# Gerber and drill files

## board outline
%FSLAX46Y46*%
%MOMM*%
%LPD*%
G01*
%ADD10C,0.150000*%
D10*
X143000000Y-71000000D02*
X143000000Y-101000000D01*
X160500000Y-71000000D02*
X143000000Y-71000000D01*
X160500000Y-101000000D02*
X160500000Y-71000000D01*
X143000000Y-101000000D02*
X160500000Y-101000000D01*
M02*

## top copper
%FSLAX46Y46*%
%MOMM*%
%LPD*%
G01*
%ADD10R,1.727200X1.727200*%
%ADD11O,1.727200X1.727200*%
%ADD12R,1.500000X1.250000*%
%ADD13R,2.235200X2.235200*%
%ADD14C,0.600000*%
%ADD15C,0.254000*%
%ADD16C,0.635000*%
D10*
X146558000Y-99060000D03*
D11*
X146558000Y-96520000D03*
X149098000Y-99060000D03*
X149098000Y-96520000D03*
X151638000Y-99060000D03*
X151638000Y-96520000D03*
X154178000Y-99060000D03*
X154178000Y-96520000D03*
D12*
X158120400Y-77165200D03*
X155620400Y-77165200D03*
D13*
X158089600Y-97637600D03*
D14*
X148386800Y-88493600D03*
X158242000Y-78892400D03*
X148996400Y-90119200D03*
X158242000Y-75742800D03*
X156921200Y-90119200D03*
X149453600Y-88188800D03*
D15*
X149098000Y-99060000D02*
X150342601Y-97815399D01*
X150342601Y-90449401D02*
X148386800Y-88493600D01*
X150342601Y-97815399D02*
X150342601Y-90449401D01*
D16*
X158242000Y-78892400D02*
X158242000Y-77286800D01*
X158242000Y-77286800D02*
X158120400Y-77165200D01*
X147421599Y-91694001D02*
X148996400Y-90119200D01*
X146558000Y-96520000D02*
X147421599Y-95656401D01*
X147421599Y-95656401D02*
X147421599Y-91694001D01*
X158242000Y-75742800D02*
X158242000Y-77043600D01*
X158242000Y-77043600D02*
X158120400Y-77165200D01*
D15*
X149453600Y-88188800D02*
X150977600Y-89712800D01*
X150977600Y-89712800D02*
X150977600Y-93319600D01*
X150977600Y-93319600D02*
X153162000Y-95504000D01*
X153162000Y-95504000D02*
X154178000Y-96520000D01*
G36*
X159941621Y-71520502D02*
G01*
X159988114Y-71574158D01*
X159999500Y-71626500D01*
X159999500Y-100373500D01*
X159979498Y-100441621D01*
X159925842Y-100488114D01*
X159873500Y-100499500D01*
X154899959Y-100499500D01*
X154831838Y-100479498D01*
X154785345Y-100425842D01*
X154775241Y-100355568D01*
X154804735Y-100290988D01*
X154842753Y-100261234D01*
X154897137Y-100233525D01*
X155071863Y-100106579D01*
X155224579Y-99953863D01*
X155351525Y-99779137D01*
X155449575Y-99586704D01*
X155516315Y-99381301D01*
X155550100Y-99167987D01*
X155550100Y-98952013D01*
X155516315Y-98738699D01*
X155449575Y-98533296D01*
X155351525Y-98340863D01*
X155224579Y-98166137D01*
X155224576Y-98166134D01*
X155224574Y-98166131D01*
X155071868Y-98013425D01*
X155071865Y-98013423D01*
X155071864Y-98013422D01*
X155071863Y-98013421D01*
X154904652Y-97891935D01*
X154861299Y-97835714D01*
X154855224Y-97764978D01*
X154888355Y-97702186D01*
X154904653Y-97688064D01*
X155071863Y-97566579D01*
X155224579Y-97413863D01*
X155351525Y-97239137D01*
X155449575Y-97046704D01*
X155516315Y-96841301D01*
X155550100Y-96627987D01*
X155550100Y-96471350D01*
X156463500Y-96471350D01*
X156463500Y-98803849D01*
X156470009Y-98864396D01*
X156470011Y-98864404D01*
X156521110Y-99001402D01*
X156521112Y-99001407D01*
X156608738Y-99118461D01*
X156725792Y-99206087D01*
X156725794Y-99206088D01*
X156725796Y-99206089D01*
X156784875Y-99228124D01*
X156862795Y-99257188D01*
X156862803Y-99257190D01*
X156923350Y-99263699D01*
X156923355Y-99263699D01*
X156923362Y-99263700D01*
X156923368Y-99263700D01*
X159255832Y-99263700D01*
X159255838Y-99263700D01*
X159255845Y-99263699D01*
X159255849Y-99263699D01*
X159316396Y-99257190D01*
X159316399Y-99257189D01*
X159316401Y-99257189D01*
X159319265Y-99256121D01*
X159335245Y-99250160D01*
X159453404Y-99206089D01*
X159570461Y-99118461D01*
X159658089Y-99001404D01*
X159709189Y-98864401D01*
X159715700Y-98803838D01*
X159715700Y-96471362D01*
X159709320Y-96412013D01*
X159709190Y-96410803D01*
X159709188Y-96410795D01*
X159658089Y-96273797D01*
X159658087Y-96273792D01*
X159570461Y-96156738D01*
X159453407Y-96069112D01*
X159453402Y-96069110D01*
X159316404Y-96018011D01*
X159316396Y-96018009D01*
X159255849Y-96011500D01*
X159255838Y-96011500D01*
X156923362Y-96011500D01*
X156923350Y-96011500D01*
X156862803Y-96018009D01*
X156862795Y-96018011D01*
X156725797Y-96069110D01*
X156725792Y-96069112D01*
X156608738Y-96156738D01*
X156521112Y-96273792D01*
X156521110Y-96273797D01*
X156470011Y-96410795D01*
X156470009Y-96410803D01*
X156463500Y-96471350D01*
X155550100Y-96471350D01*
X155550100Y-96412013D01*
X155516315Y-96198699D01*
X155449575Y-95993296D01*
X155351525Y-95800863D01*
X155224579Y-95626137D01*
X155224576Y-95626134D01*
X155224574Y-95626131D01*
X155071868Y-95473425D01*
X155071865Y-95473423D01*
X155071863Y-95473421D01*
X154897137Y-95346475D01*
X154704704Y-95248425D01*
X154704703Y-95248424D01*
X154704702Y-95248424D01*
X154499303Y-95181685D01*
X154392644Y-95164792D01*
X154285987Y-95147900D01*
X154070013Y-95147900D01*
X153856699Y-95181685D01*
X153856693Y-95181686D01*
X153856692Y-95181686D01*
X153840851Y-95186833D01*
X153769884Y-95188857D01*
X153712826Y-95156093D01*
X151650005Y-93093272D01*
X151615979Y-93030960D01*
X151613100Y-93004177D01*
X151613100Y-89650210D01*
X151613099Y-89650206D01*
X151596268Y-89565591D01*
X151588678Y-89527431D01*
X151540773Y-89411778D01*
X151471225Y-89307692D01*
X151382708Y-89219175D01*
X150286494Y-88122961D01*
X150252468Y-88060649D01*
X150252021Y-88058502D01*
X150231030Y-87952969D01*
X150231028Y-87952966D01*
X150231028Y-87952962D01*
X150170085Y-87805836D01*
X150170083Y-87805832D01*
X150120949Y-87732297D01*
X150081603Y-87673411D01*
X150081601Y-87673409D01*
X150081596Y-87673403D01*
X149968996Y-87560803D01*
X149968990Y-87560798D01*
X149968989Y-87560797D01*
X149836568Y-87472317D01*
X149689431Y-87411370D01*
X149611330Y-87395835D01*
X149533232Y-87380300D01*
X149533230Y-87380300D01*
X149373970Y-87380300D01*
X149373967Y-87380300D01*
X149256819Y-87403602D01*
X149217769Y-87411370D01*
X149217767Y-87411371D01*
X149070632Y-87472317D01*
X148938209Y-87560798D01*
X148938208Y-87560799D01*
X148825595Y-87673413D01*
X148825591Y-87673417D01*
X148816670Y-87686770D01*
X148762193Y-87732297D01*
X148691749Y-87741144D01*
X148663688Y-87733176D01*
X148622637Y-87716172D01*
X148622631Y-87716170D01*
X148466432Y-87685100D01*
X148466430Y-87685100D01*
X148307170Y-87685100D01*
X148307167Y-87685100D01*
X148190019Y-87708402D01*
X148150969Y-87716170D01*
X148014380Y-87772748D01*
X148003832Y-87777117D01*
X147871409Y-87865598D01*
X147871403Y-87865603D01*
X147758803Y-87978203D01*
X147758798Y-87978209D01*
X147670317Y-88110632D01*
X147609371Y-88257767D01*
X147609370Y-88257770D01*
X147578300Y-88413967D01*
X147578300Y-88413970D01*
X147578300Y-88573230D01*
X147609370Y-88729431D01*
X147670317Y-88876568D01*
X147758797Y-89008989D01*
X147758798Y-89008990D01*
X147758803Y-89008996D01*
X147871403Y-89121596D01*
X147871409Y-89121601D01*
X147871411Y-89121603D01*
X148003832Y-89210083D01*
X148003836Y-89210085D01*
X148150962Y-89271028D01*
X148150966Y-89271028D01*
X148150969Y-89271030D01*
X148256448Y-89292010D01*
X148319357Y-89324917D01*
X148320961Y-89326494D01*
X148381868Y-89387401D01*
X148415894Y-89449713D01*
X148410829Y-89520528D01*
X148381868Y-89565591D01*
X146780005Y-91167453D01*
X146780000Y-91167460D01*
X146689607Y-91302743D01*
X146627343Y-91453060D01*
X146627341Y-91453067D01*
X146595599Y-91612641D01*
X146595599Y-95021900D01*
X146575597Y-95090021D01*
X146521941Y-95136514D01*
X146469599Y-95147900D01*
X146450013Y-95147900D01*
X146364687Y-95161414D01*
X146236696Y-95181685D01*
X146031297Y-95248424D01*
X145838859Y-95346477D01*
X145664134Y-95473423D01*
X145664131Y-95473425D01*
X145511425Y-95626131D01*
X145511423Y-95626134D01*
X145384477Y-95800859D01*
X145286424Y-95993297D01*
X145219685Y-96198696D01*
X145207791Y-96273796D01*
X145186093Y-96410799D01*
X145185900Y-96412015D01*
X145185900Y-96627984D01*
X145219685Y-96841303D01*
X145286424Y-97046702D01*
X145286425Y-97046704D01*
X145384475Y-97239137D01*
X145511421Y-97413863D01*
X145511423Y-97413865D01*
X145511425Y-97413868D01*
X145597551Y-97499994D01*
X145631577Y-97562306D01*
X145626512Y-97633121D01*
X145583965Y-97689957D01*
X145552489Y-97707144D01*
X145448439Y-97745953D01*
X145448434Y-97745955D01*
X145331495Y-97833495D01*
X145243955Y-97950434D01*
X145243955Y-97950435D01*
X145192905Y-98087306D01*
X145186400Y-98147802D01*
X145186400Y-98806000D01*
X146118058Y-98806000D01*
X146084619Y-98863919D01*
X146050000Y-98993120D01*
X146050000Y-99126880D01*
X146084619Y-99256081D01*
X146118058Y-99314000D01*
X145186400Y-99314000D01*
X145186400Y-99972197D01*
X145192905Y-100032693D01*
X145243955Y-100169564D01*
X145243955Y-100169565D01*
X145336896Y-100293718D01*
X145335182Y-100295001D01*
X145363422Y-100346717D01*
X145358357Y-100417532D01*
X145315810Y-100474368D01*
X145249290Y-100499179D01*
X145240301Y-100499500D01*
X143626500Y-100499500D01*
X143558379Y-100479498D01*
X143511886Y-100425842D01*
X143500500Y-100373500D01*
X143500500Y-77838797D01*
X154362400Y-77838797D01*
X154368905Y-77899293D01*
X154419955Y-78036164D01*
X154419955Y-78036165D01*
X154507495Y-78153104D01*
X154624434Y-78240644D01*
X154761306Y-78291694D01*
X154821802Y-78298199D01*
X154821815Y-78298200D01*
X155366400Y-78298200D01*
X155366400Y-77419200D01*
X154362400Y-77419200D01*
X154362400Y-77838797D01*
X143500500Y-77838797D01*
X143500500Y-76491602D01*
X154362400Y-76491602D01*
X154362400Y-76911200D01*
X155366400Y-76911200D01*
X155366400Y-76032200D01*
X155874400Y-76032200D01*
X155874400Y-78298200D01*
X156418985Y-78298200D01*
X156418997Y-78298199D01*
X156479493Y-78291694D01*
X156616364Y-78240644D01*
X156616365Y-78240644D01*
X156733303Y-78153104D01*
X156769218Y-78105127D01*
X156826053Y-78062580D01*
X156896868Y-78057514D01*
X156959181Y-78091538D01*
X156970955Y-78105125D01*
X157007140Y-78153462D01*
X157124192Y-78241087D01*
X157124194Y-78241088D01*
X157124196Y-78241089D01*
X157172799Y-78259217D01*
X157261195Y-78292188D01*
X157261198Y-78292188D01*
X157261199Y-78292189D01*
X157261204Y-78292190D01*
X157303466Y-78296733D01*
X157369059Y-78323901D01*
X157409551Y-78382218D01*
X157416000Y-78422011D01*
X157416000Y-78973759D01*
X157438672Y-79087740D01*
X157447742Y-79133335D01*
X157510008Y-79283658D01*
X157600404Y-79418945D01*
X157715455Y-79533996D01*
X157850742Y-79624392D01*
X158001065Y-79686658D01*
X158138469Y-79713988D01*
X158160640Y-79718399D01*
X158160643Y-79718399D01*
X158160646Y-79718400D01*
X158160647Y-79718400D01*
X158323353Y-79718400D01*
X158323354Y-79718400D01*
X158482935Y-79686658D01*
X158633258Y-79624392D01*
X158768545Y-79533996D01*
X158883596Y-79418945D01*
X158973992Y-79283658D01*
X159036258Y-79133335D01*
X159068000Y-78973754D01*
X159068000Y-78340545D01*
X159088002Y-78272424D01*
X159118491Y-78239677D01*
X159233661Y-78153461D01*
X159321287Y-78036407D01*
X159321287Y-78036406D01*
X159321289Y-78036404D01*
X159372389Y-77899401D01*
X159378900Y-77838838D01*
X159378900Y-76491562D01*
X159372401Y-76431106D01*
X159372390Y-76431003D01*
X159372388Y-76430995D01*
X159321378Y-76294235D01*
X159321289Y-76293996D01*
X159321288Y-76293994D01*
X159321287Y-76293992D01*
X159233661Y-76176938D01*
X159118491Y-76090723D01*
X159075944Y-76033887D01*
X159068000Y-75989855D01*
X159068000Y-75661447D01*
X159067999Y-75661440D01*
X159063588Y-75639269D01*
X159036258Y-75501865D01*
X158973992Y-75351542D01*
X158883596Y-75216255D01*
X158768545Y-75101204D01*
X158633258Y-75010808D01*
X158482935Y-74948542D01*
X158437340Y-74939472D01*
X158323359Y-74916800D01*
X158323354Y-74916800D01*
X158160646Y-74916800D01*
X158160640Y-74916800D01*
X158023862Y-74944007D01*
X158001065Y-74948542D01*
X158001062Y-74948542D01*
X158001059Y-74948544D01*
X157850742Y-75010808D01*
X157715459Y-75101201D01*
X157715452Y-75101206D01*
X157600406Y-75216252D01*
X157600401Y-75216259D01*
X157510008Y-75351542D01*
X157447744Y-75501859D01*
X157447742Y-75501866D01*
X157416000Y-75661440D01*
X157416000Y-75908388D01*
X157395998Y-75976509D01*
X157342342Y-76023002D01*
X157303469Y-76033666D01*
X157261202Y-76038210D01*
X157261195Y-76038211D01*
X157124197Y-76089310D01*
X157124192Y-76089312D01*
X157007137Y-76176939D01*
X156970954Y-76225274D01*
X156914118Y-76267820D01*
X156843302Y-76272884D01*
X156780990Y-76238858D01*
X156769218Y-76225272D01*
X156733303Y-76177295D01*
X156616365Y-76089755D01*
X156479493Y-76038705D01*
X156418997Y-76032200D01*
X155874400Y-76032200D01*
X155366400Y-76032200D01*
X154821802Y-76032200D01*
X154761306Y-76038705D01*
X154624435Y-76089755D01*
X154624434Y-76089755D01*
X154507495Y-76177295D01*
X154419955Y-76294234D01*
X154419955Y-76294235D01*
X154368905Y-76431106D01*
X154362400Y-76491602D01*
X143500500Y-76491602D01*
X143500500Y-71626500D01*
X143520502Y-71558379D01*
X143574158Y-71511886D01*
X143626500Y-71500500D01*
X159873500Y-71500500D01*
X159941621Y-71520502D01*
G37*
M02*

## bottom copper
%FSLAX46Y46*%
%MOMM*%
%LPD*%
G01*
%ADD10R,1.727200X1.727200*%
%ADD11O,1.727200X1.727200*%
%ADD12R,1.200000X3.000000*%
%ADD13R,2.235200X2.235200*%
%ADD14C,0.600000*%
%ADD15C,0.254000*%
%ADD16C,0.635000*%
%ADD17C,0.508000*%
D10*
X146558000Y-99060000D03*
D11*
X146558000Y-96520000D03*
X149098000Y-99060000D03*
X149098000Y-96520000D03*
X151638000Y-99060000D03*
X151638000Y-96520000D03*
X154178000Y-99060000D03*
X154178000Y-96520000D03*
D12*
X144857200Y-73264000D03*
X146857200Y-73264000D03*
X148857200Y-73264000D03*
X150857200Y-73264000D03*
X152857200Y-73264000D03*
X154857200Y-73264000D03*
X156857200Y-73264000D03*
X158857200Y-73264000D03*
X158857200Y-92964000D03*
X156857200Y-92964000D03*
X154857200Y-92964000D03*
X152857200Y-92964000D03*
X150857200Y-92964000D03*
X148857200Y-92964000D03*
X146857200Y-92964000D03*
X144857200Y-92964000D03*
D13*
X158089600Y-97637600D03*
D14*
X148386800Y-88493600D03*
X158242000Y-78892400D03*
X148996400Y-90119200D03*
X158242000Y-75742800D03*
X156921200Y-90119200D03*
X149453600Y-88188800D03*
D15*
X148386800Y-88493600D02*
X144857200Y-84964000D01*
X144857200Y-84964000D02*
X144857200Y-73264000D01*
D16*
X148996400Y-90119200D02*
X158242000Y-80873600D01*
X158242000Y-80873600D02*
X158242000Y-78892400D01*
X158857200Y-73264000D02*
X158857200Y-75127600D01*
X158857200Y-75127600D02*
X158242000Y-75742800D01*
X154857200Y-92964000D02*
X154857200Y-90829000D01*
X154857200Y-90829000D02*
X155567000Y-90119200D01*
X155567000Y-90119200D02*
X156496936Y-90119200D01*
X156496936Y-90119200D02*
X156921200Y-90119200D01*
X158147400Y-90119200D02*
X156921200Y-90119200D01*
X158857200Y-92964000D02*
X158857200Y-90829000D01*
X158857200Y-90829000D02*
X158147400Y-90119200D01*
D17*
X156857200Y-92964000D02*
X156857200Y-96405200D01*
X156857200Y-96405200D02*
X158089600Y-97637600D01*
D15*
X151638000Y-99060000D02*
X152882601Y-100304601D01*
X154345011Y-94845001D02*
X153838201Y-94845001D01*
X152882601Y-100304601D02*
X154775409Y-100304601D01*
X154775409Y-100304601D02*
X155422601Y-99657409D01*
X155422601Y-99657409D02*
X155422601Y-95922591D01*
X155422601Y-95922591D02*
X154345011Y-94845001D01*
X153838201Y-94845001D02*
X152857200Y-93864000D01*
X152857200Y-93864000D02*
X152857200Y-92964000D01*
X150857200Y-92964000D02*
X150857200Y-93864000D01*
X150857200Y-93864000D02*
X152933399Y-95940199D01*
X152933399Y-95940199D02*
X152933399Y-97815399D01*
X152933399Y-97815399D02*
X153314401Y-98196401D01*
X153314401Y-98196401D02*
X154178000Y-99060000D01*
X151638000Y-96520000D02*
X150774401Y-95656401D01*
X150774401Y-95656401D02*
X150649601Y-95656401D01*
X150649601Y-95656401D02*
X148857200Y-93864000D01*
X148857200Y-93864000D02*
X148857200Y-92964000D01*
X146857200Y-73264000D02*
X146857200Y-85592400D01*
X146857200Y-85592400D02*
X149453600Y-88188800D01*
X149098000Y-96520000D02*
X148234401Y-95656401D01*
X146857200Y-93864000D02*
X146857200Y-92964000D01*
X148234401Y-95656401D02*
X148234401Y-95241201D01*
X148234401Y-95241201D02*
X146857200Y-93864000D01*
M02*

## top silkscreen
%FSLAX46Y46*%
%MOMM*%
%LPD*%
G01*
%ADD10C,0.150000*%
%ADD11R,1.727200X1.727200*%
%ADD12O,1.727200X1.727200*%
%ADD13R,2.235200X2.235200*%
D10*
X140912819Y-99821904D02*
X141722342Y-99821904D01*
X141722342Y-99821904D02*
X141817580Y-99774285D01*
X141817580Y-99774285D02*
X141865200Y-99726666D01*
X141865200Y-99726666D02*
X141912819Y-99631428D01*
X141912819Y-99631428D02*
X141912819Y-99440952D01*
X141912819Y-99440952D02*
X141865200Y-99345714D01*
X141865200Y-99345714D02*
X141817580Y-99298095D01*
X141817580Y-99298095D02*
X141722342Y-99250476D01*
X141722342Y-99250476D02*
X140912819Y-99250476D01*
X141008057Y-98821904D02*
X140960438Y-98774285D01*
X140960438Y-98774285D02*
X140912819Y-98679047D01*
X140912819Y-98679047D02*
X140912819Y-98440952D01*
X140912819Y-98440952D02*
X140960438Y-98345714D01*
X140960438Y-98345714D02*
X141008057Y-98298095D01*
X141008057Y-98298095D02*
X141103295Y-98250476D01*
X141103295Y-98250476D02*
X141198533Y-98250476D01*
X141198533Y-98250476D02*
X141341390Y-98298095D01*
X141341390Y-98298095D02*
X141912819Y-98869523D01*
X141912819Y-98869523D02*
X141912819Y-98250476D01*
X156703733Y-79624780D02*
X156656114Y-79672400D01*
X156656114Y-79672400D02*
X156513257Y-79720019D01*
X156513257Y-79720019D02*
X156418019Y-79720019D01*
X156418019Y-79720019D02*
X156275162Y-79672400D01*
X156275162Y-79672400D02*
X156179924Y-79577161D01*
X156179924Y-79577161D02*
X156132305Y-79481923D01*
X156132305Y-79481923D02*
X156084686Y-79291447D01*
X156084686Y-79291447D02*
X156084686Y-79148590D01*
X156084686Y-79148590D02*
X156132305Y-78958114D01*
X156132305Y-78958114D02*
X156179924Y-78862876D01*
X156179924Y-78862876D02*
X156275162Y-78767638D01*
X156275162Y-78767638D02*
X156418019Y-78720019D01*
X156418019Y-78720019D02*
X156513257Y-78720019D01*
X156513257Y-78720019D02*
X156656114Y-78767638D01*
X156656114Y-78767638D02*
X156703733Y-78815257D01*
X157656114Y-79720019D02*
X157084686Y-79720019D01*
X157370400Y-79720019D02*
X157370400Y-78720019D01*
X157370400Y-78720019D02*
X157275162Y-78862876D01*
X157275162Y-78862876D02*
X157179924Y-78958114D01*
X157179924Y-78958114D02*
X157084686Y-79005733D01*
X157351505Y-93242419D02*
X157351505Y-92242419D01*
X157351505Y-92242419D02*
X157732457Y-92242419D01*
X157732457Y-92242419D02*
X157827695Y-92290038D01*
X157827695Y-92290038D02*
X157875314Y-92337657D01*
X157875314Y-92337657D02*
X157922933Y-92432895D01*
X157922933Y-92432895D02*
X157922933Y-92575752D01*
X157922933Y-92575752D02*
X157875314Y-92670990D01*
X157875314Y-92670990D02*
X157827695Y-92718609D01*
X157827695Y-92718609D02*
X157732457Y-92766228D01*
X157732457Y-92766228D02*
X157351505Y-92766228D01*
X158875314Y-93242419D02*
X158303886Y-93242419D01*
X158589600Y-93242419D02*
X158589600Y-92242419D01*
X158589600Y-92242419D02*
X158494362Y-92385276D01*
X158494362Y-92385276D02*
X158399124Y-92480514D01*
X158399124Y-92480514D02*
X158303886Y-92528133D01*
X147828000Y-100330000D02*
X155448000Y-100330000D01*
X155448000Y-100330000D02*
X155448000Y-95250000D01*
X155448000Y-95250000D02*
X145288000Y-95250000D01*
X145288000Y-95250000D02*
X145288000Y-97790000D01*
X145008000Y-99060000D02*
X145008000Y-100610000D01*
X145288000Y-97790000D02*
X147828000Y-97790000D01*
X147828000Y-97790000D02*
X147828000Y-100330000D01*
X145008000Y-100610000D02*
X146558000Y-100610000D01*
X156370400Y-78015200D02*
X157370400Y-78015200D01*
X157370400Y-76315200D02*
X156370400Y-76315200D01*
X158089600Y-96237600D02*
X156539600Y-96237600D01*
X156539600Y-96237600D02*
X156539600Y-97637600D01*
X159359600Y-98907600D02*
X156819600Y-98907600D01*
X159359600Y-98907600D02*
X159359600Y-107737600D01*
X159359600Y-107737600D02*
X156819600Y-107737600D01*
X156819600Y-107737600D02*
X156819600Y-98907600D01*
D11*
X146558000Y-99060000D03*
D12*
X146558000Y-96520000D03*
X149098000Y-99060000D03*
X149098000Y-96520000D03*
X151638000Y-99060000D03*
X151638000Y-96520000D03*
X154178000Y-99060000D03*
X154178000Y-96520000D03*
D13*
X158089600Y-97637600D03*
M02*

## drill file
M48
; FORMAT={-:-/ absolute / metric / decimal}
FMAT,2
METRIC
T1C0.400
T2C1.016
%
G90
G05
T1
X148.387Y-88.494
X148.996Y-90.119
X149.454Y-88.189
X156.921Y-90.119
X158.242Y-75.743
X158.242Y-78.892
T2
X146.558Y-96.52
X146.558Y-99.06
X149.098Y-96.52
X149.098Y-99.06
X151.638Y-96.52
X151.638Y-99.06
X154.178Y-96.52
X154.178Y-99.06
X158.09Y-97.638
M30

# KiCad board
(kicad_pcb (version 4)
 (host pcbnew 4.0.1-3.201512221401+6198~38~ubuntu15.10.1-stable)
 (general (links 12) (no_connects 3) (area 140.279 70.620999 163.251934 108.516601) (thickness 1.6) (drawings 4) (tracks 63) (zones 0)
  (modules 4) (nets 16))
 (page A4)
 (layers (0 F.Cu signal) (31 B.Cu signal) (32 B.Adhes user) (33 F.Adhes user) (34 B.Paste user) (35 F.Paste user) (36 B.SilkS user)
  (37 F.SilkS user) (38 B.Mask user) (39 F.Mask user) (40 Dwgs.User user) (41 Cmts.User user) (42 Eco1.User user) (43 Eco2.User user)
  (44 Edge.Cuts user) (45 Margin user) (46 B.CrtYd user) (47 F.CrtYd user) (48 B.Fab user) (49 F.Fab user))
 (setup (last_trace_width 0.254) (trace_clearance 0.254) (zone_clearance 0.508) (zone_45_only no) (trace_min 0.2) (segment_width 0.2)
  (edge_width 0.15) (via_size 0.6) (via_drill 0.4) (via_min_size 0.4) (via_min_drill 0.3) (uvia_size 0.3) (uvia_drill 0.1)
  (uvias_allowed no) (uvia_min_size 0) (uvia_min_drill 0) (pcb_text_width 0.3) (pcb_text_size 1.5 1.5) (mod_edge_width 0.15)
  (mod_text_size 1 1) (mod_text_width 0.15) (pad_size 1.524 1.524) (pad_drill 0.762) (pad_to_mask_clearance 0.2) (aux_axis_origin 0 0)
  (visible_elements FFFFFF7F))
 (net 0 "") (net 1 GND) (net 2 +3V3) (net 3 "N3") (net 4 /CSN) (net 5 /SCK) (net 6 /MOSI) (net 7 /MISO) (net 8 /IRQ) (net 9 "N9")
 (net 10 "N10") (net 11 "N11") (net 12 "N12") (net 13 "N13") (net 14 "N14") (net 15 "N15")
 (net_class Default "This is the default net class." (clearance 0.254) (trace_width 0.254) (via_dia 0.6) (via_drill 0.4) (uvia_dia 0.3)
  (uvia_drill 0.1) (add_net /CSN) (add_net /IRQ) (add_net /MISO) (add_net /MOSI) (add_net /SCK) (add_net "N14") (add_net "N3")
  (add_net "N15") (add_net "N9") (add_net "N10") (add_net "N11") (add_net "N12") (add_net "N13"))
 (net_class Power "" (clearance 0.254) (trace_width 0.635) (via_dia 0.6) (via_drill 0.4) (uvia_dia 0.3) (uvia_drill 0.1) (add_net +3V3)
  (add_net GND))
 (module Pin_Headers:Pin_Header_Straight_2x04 (layer F.Cu) (at 146.558 99.06 90)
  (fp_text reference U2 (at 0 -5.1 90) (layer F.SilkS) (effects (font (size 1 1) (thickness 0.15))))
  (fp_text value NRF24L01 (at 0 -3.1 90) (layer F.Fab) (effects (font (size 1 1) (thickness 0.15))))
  (fp_line (start -1.27 1.27) (end -1.27 8.89) (layer F.SilkS) (width 0.15))
  (fp_line (start -1.27 8.89) (end 3.81 8.89) (layer F.SilkS) (width 0.15))
  (fp_line (start 3.81 8.89) (end 3.81 -1.27) (layer F.SilkS) (width 0.15))
  (fp_line (start 3.81 -1.27) (end 1.27 -1.27) (layer F.SilkS) (width 0.15))
  (fp_line (start 0 -1.55) (end -1.55 -1.55) (layer F.SilkS) (width 0.15))
  (fp_line (start 1.27 -1.27) (end 1.27 1.27) (layer F.SilkS) (width 0.15))
  (fp_line (start 1.27 1.27) (end -1.27 1.27) (layer F.SilkS) (width 0.15))
  (fp_line (start -1.55 -1.55) (end -1.55 0) (layer F.SilkS) (width 0.15))
  (pad 1 thru_hole rect (at 0 0 90) (size 1.7272 1.7272) (drill 1.016) (layers *.Cu *.Mask F.SilkS) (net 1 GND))
  (pad 2 thru_hole oval (at 2.54 0 90) (size 1.7272 1.7272) (drill 1.016) (layers *.Cu *.Mask F.SilkS) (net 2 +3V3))
  (pad 3 thru_hole oval (at 0 2.54 90) (size 1.7272 1.7272) (drill 1.016) (layers *.Cu *.Mask F.SilkS) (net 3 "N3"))
  (pad 4 thru_hole oval (at 2.54 2.54 90) (size 1.7272 1.7272) (drill 1.016) (layers *.Cu *.Mask F.SilkS) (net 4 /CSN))
  (pad 5 thru_hole oval (at 0 5.08 90) (size 1.7272 1.7272) (drill 1.016) (layers *.Cu *.Mask F.SilkS) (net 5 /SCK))
  (pad 6 thru_hole oval (at 2.54 5.08 90) (size 1.7272 1.7272) (drill 1.016) (layers *.Cu *.Mask F.SilkS) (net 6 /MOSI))
  (pad 7 thru_hole oval (at 0 7.62 90) (size 1.7272 1.7272) (drill 1.016) (layers *.Cu *.Mask F.SilkS) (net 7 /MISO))
  (pad 8 thru_hole oval (at 2.54 7.62 90) (size 1.7272 1.7272) (drill 1.016) (layers *.Cu *.Mask F.SilkS) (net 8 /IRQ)))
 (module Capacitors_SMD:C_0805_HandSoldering (layer F.Cu) (at 156.8704 77.1652 180)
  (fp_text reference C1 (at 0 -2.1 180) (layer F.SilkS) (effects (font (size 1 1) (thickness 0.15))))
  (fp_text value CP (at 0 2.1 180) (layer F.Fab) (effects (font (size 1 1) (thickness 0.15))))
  (fp_line (start 0.5 -0.85) (end -0.5 -0.85) (layer F.SilkS) (width 0.15))
  (fp_line (start -0.5 0.85) (end 0.5 0.85) (layer F.SilkS) (width 0.15))
  (pad 1 smd rect (at -1.25 0 180) (size 1.5 1.25) (layers F.Cu F.Paste F.Mask) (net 2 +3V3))
  (pad 2 smd rect (at 1.25 0 180) (size 1.5 1.25) (layers F.Cu F.Paste F.Mask) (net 1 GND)))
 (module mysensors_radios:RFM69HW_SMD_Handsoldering (layer B.Cu) (at 144.8572 74.664 270)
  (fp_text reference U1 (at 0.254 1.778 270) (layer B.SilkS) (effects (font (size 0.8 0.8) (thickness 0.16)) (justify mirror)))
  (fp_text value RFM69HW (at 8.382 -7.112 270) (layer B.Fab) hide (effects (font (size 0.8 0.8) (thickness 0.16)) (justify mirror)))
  (pad 1 smd rect (at -1.4 0 270) (size 3 1.2) (layers B.Cu B.Paste B.Mask) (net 3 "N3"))
  (pad 2 smd rect (at -1.4 -2 270) (size 3 1.2) (layers B.Cu B.Paste B.Mask) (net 8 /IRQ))
  (pad 3 smd rect (at -1.4 -4 270) (size 3 1.2) (layers B.Cu B.Paste B.Mask) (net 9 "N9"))
  (pad 4 smd rect (at -1.4 -6 270) (size 3 1.2) (layers B.Cu B.Paste B.Mask) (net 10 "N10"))
  (pad 5 smd rect (at -1.4 -8 270) (size 3 1.2) (layers B.Cu B.Paste B.Mask) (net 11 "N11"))
  (pad 6 smd rect (at -1.4 -10 270) (size 3 1.2) (layers B.Cu B.Paste B.Mask) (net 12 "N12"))
  (pad 7 smd rect (at -1.4 -12 270) (size 3 1.2) (layers B.Cu B.Paste B.Mask) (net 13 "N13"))
  (pad 8 smd rect (at -1.4 -14 270) (size 3 1.2) (layers B.Cu B.Paste B.Mask) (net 2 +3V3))
  (pad 9 smd rect (at 18.3 -14 270) (size 3 1.2) (layers B.Cu B.Paste B.Mask) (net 1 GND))
  (pad 10 smd rect (at 18.3 -12 270) (size 3 1.2) (layers B.Cu B.Paste B.Mask) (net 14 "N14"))
  (pad 11 smd rect (at 18.3 -10 270) (size 3 1.2) (layers B.Cu B.Paste B.Mask) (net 1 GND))
  (pad 12 smd rect (at 18.3 -8 270) (size 3 1.2) (layers B.Cu B.Paste B.Mask) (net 5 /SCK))
  (pad 13 smd rect (at 18.3 -6 270) (size 3 1.2) (layers B.Cu B.Paste B.Mask) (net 7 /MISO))
  (pad 14 smd rect (at 18.3 -4 270) (size 3 1.2) (layers B.Cu B.Paste B.Mask) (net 6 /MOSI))
  (pad 15 smd rect (at 18.3 -2 270) (size 3 1.2) (layers B.Cu B.Paste B.Mask) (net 4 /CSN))
  (pad 16 smd rect (at 18.3 0 270) (size 3 1.2) (layers B.Cu B.Paste B.Mask) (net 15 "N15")))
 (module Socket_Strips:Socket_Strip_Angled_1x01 (layer F.Cu) (at 158.0896 97.6376)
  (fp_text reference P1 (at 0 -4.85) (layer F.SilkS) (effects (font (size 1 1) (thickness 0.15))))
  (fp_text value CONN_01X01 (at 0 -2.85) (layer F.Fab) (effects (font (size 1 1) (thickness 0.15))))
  (fp_line (start 0 -1.4) (end -1.55 -1.4) (layer F.SilkS) (width 0.15))
  (fp_line (start -1.55 -1.4) (end -1.55 0) (layer F.SilkS) (width 0.15))
  (fp_line (start 1.27 1.27) (end -1.27 1.27) (layer F.SilkS) (width 0.15))
  (fp_line (start 1.27 1.27) (end 1.27 10.1) (layer F.SilkS) (width 0.15))
  (fp_line (start 1.27 10.1) (end -1.27 10.1) (layer F.SilkS) (width 0.15))
  (fp_line (start -1.27 10.1) (end -1.27 1.27) (layer F.SilkS) (width 0.15))
  (pad 1 thru_hole rect (at 0 0) (size 2.2352 2.2352) (drill 1.016) (layers *.Cu *.Mask F.SilkS) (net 14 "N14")))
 (gr_line (start 143 71) (end 143 101) (layer Edge.Cuts) (width 0.15))
 (gr_line (start 160.5 71) (end 143 71) (layer Edge.Cuts) (width 0.15))
 (gr_line (start 160.5 101) (end 160.5 71) (layer Edge.Cuts) (width 0.15))
 (gr_line (start 143 101) (end 160.5 101) (layer Edge.Cuts) (width 0.15))
 (segment (start 143 71) (end 143 101.5) (width 0.25) (layer Dwgs.User) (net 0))
 (segment (start 160.5 71) (end 143 71) (width 0.25) (layer Dwgs.User) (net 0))
 (segment (start 160.5 101) (end 160.5 71) (width 0.25) (layer Dwgs.User) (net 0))
 (segment (start 143 101) (end 160.5 101) (width 0.25) (layer Dwgs.User) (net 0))
 (segment (start 146.3675 101.6635) (end 158.496 101.6635) (width 0.25) (layer Dwgs.User) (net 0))
 (segment (start 148.3868 88.4936) (end 144.8572 84.964) (width 0.254) (layer B.Cu) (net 3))
 (segment (start 144.8572 84.964) (end 144.8572 73.264) (width 0.254) (layer B.Cu) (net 3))
 (segment (start 149.098 99.06) (end 150.342601 97.815399) (width 0.254) (layer F.Cu) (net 3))
 (segment (start 150.342601 90.449401) (end 148.3868 88.4936) (width 0.254) (layer F.Cu) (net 3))
 (segment (start 150.342601 97.815399) (end 150.342601 90.449401) (width 0.254) (layer F.Cu) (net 3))
 (via (at 148.3868 88.4936) (size 0.6) (drill 0.4) (layers F.Cu B.Cu) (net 3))
 (segment (start 158.242 78.8924) (end 158.242 77.2868) (width 0.635) (layer F.Cu) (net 2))
 (segment (start 158.242 77.2868) (end 158.1204 77.1652) (width 0.635) (layer F.Cu) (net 2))
 (segment (start 148.9964 90.1192) (end 158.242 80.8736) (width 0.635) (layer B.Cu) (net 2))
 (via (at 158.242 78.8924) (size 0.6) (drill 0.4) (layers F.Cu B.Cu) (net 2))
 (segment (start 158.242 80.8736) (end 158.242 78.8924) (width 0.635) (layer B.Cu) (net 2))
 (segment (start 147.421599 91.694001) (end 148.9964 90.1192) (width 0.635) (layer F.Cu) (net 2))
 (via (at 148.9964 90.1192) (size 0.6) (drill 0.4) (layers F.Cu B.Cu) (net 2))
 (segment (start 146.558 96.52) (end 147.421599 95.656401) (width 0.635) (layer F.Cu) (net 2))
 (segment (start 147.421599 95.656401) (end 147.421599 91.694001) (width 0.635) (layer F.Cu) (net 2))
 (segment (start 158.242 75.7428) (end 158.242 77.0436) (width 0.635) (layer F.Cu) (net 2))
 (segment (start 158.242 77.0436) (end 158.1204 77.1652) (width 0.635) (layer F.Cu) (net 2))
 (segment (start 158.8572 73.264) (end 158.8572 75.1276) (width 0.635) (layer B.Cu) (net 2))
 (segment (start 158.8572 75.1276) (end 158.242 75.7428) (width 0.635) (layer B.Cu) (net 2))
 (via (at 158.242 75.7428) (size 0.6) (drill 0.4) (layers F.Cu B.Cu) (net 2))
 (segment (start 154.8572 92.964) (end 154.8572 90.829) (width 0.635) (layer B.Cu) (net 1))
 (segment (start 154.8572 90.829) (end 155.567 90.1192) (width 0.635) (layer B.Cu) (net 1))
 (segment (start 155.567 90.1192) (end 156.496936 90.1192) (width 0.635) (layer B.Cu) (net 1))
 (segment (start 156.496936 90.1192) (end 156.9212 90.1192) (width 0.635) (layer B.Cu) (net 1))
 (segment (start 158.1474 90.1192) (end 156.9212 90.1192) (width 0.635) (layer B.Cu) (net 1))
 (via (at 156.9212 90.1192) (size 0.6) (drill 0.4) (layers F.Cu B.Cu) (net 1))
 (segment (start 158.8572 92.964) (end 158.8572 90.829) (width 0.635) (layer B.Cu) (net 1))
 (segment (start 158.8572 90.829) (end 158.1474 90.1192) (width 0.635) (layer B.Cu) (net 1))
 (segment (start 156.8572 92.964) (end 156.8572 96.4052) (width 0.508) (layer B.Cu) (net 14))
 (segment (start 156.8572 96.4052) (end 158.0896 97.6376) (width 0.508) (layer B.Cu) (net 14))
 (segment (start 151.638 99.06) (end 152.882601 100.304601) (width 0.254) (layer B.Cu) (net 5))
 (segment (start 154.345011 94.845001) (end 153.838201 94.845001) (width 0.254) (layer B.Cu) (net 5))
 (segment (start 152.882601 100.304601) (end 154.775409 100.304601) (width 0.254) (layer B.Cu) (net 5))
 (segment (start 154.775409 100.304601) (end 155.422601 99.657409) (width 0.254) (layer B.Cu) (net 5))
 (segment (start 155.422601 99.657409) (end 155.422601 95.922591) (width 0.254) (layer B.Cu) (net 5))
 (segment (start 155.422601 95.922591) (end 154.345011 94.845001) (width 0.254) (layer B.Cu) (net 5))
 (segment (start 153.838201 94.845001) (end 152.8572 93.864) (width 0.254) (layer B.Cu) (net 5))
 (segment (start 152.8572 93.864) (end 152.8572 92.964) (width 0.254) (layer B.Cu) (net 5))
 (segment (start 150.8572 92.964) (end 150.8572 93.864) (width 0.254) (layer B.Cu) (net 7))
 (segment (start 150.8572 93.864) (end 152.933399 95.940199) (width 0.254) (layer B.Cu) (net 7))
 (segment (start 152.933399 95.940199) (end 152.933399 97.815399) (width 0.254) (layer B.Cu) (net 7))
 (segment (start 152.933399 97.815399) (end 153.314401 98.196401) (width 0.254) (layer B.Cu) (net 7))
 (segment (start 153.314401 98.196401) (end 154.178 99.06) (width 0.254) (layer B.Cu) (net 7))
 (segment (start 151.638 96.52) (end 150.774401 95.656401) (width 0.254) (layer B.Cu) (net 6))
 (segment (start 150.774401 95.656401) (end 150.649601 95.656401) (width 0.254) (layer B.Cu) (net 6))
 (segment (start 150.649601 95.656401) (end 148.8572 93.864) (width 0.254) (layer B.Cu) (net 6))
 (segment (start 148.8572 93.864) (end 148.8572 92.964) (width 0.254) (layer B.Cu) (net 6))
 (segment (start 149.4536 88.1888) (end 150.9776 89.7128) (width 0.254) (layer F.Cu) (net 8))
 (segment (start 150.9776 89.7128) (end 150.9776 93.3196) (width 0.254) (layer F.Cu) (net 8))
 (segment (start 150.9776 93.3196) (end 153.162 95.504) (width 0.254) (layer F.Cu) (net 8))
 (segment (start 153.162 95.504) (end 154.178 96.52) (width 0.254) (layer F.Cu) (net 8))
 (segment (start 146.8572 73.264) (end 146.8572 85.5924) (width 0.254) (layer B.Cu) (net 8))
 (segment (start 146.8572 85.5924) (end 149.4536 88.1888) (width 0.254) (layer B.Cu) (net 8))
 (via (at 149.4536 88.1888) (size 0.6) (drill 0.4) (layers F.Cu B.Cu) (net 8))
 (segment (start 149.098 96.52) (end 148.234401 95.656401) (width 0.254) (layer B.Cu) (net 4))
 (segment (start 146.8572 93.864) (end 146.8572 92.964) (width 0.254) (layer B.Cu) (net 4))
 (segment (start 148.234401 95.656401) (end 148.234401 95.241201) (width 0.254) (layer B.Cu) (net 4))
 (segment (start 148.234401 95.241201) (end 146.8572 93.864) (width 0.254) (layer B.Cu) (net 4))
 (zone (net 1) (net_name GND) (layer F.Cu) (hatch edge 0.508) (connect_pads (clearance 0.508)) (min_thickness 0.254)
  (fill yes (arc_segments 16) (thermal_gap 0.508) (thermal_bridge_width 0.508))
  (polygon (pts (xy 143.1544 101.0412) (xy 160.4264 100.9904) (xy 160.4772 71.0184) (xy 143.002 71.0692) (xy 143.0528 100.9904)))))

